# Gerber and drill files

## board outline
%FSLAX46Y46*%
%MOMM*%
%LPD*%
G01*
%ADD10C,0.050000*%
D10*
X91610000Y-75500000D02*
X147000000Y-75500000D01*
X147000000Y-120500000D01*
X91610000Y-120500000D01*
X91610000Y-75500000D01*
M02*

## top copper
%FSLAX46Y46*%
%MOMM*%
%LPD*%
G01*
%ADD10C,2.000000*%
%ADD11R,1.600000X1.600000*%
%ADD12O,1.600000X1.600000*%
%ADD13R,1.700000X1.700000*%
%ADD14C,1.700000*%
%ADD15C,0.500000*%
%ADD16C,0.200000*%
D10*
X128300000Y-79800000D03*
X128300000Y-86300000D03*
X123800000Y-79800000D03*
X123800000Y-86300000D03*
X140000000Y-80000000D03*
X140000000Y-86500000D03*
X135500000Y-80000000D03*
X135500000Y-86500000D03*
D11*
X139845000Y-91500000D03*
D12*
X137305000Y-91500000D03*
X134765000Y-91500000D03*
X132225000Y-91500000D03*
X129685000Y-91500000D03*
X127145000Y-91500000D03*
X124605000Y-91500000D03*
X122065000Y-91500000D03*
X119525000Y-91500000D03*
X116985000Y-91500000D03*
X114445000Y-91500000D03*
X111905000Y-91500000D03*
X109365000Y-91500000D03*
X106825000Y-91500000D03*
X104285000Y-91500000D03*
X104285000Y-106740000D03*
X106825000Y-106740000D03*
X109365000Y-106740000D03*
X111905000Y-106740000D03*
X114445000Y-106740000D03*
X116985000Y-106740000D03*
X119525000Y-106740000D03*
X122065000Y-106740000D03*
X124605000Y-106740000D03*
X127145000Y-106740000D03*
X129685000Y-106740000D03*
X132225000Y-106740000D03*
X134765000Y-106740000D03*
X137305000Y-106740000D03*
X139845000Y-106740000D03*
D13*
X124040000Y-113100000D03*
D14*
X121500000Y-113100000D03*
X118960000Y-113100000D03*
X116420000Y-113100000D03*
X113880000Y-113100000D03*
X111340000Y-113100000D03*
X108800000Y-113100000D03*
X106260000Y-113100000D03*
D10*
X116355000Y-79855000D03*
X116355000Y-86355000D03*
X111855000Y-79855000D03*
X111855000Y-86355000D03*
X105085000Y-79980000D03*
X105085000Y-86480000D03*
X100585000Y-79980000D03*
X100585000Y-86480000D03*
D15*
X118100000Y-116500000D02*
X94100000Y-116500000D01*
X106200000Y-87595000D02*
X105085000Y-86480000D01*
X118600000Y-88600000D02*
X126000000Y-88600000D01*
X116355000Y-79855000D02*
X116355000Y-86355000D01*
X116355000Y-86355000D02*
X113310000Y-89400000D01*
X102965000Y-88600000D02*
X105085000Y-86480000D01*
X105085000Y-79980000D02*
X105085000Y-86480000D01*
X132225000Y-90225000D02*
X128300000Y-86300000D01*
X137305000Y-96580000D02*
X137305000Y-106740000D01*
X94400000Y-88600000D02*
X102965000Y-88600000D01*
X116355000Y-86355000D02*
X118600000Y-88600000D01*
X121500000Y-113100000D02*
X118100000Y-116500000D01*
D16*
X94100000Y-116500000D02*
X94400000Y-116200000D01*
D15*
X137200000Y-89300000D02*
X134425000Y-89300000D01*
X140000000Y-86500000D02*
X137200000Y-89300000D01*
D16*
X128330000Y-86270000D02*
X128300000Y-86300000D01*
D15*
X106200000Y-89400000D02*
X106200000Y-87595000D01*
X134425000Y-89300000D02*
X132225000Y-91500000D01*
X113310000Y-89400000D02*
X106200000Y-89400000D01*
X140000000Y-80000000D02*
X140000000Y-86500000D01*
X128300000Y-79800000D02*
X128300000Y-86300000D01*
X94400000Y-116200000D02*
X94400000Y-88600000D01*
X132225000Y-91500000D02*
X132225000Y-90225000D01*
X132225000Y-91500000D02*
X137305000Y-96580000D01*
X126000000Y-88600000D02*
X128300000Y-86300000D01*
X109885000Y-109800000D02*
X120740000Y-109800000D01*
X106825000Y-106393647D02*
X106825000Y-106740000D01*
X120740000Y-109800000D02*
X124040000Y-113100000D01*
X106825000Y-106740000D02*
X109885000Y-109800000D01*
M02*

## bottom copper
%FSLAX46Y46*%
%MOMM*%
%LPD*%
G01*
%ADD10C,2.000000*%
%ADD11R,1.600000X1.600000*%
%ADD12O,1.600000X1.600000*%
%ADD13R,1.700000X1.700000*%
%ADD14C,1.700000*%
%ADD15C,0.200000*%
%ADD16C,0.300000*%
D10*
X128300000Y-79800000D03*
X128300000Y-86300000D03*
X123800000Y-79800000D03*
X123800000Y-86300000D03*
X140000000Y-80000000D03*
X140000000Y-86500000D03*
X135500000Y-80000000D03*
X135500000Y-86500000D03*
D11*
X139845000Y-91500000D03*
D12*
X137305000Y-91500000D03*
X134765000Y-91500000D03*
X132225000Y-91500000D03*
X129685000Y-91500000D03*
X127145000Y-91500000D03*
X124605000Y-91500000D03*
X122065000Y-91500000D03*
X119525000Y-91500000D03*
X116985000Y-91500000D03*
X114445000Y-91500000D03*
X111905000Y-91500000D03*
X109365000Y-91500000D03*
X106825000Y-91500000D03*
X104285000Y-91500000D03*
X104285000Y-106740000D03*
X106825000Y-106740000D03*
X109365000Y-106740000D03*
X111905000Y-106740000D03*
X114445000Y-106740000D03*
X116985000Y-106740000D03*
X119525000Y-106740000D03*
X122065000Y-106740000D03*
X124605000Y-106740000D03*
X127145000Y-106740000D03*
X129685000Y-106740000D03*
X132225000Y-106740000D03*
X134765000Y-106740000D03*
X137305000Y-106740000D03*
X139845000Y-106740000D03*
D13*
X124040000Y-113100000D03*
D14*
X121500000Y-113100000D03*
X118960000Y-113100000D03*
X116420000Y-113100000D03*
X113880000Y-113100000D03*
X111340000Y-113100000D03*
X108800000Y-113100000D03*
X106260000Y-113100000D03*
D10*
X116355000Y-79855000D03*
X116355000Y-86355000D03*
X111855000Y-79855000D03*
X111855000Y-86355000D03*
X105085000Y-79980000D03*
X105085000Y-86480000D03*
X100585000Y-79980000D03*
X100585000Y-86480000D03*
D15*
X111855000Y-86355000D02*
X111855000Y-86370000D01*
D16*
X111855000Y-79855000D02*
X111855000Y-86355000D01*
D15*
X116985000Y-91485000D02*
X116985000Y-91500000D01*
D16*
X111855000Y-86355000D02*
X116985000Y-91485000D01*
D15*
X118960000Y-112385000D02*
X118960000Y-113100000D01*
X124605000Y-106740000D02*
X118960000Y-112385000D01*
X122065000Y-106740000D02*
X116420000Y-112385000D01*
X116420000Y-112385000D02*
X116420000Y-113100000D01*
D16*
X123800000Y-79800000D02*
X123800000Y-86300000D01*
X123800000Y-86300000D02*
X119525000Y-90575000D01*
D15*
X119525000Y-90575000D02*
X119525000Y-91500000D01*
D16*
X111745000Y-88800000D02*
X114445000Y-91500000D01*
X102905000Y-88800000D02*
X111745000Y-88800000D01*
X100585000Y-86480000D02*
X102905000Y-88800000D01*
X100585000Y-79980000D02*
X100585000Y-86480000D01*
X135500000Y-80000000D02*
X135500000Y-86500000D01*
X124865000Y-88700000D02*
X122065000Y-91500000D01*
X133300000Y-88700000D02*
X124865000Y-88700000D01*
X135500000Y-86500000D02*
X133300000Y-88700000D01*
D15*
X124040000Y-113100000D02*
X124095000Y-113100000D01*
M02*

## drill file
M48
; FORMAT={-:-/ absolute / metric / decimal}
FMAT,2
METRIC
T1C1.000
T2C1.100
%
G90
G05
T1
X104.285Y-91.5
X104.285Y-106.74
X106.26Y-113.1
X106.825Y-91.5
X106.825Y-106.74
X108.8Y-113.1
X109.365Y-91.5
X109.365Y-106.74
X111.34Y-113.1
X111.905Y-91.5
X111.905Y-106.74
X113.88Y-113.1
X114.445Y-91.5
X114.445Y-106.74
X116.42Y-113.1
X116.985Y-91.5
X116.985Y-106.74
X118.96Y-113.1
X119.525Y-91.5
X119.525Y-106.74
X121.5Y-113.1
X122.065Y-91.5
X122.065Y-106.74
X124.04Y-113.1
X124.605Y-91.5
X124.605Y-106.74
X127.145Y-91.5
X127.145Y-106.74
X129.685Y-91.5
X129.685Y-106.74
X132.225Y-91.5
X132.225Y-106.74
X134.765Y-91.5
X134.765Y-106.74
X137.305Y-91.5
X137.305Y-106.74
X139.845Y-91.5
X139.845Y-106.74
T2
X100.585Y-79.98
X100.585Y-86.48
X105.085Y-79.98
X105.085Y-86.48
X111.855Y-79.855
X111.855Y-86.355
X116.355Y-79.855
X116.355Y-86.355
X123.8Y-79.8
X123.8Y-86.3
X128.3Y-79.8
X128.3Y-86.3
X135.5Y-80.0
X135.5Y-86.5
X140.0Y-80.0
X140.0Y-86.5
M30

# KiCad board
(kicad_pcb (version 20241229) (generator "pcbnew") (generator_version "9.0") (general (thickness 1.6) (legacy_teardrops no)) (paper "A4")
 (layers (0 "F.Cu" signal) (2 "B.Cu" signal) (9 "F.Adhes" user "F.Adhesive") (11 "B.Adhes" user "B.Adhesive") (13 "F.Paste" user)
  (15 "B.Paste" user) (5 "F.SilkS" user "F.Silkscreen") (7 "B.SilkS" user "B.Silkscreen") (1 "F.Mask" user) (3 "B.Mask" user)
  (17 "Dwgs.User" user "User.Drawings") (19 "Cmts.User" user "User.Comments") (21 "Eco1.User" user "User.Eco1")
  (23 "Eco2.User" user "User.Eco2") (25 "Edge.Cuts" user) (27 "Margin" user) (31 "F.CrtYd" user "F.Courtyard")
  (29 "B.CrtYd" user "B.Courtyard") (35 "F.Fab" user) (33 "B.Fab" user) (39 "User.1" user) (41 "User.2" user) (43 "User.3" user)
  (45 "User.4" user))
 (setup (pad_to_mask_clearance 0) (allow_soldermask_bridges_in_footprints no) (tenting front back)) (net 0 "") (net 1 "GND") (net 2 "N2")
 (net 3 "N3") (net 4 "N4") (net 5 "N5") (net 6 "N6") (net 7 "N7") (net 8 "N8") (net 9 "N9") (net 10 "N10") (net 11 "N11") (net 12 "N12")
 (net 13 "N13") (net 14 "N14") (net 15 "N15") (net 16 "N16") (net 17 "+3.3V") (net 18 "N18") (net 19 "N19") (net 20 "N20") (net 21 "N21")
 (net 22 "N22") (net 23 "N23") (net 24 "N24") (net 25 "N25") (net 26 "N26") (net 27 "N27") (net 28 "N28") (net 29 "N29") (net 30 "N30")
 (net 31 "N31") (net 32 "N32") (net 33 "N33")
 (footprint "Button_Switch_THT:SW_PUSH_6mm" (layer "F.Cu") (at 128.3 79.8 -90)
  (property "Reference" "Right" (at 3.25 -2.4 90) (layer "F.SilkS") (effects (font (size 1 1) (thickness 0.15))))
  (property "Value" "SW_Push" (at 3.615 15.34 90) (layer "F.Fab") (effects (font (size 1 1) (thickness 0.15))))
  (pad "1" thru_hole circle (at 0 0) (size 2 2) (drill 1.1) (layers "*.Cu" "*.Mask") (remove_unused_layers no) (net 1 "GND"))
  (pad "1" thru_hole circle (at 6.5 0) (size 2 2) (drill 1.1) (layers "*.Cu" "*.Mask") (remove_unused_layers no) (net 1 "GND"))
  (pad "2" thru_hole circle (at 0 4.5) (size 2 2) (drill 1.1) (layers "*.Cu" "*.Mask") (remove_unused_layers no) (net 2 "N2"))
  (pad "2" thru_hole circle (at 6.5 4.5) (size 2 2) (drill 1.1) (layers "*.Cu" "*.Mask") (remove_unused_layers no) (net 2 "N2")))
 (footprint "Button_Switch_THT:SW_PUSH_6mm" (layer "F.Cu") (at 140 80 -90)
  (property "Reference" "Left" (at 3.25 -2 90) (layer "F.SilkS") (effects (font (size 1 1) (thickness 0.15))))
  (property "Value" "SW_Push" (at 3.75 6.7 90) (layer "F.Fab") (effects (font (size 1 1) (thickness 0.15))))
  (pad "1" thru_hole circle (at 0 0) (size 2 2) (drill 1.1) (layers "*.Cu" "*.Mask") (remove_unused_layers no) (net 1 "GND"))
  (pad "1" thru_hole circle (at 6.5 0) (size 2 2) (drill 1.1) (layers "*.Cu" "*.Mask") (remove_unused_layers no) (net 1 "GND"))
  (pad "2" thru_hole circle (at 0 4.5) (size 2 2) (drill 1.1) (layers "*.Cu" "*.Mask") (remove_unused_layers no) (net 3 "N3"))
  (pad "2" thru_hole circle (at 6.5 4.5) (size 2 2) (drill 1.1) (layers "*.Cu" "*.Mask") (remove_unused_layers no) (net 3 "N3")))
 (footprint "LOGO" (layer "F.Cu") (at 135.8138 114.7318)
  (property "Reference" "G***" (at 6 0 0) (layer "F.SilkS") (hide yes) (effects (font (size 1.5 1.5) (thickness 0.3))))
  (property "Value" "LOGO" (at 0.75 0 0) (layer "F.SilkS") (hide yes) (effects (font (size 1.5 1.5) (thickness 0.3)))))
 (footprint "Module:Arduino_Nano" (layer "F.Cu") (at 139.845 91.5 -90)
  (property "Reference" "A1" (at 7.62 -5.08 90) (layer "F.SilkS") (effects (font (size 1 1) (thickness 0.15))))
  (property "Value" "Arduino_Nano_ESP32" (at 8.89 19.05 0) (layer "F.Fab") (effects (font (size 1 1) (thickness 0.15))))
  (pad "1" thru_hole rect (at 0 0 270) (size 1.6 1.6) (drill 1) (layers "*.Cu" "*.Mask") (remove_unused_layers no) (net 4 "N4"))
  (pad "2" thru_hole oval (at 0 2.54 270) (size 1.6 1.6) (drill 1) (layers "*.Cu" "*.Mask") (remove_unused_layers no) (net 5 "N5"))
  (pad "3" thru_hole oval (at 0 5.08 270) (size 1.6 1.6) (drill 1) (layers "*.Cu" "*.Mask") (remove_unused_layers no) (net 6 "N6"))
  (pad "4" thru_hole oval (at 0 7.62 270) (size 1.6 1.6) (drill 1) (layers "*.Cu" "*.Mask") (remove_unused_layers no) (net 1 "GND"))
  (pad "5" thru_hole oval (at 0 10.16 270) (size 1.6 1.6) (drill 1) (layers "*.Cu" "*.Mask") (remove_unused_layers no) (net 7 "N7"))
  (pad "6" thru_hole oval (at 0 12.7 270) (size 1.6 1.6) (drill 1) (layers "*.Cu" "*.Mask") (remove_unused_layers no) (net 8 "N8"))
  (pad "7" thru_hole oval (at 0 15.24 270) (size 1.6 1.6) (drill 1) (layers "*.Cu" "*.Mask") (remove_unused_layers no) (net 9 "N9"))
  (pad "8" thru_hole oval (at 0 17.78 270) (size 1.6 1.6) (drill 1) (layers "*.Cu" "*.Mask") (remove_unused_layers no) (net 3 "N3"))
  (pad "9" thru_hole oval (at 0 20.32 270) (size 1.6 1.6) (drill 1) (layers "*.Cu" "*.Mask") (remove_unused_layers no) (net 2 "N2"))
  (pad "10" thru_hole oval (at 0 22.86 270) (size 1.6 1.6) (drill 1) (layers "*.Cu" "*.Mask") (remove_unused_layers no) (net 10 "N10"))
  (pad "11" thru_hole oval (at 0 25.4 270) (size 1.6 1.6) (drill 1) (layers "*.Cu" "*.Mask") (remove_unused_layers no) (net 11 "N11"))
  (pad "12" thru_hole oval (at 0 27.94 270) (size 1.6 1.6) (drill 1) (layers "*.Cu" "*.Mask") (remove_unused_layers no) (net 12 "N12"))
  (pad "13" thru_hole oval (at 0 30.48 270) (size 1.6 1.6) (drill 1) (layers "*.Cu" "*.Mask") (remove_unused_layers no) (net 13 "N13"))
  (pad "14" thru_hole oval (at 0 33.02 270) (size 1.6 1.6) (drill 1) (layers "*.Cu" "*.Mask") (remove_unused_layers no) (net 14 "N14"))
  (pad "15" thru_hole oval (at 0 35.56 270) (size 1.6 1.6) (drill 1) (layers "*.Cu" "*.Mask") (remove_unused_layers no) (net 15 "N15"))
  (pad "16" thru_hole oval (at 15.24 35.56 270) (size 1.6 1.6) (drill 1) (layers "*.Cu" "*.Mask") (remove_unused_layers no) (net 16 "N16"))
  (pad "17" thru_hole oval (at 15.24 33.02 270) (size 1.6 1.6) (drill 1) (layers "*.Cu" "*.Mask") (remove_unused_layers no) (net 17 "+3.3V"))
  (pad "18" thru_hole oval (at 15.24 30.48 270) (size 1.6 1.6) (drill 1) (layers "*.Cu" "*.Mask") (remove_unused_layers no) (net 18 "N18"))
  (pad "19" thru_hole oval (at 15.24 27.94 270) (size 1.6 1.6) (drill 1) (layers "*.Cu" "*.Mask") (remove_unused_layers no) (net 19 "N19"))
  (pad "20" thru_hole oval (at 15.24 25.4 270) (size 1.6 1.6) (drill 1) (layers "*.Cu" "*.Mask") (remove_unused_layers no) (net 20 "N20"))
  (pad "21" thru_hole oval (at 15.24 22.86 270) (size 1.6 1.6) (drill 1) (layers "*.Cu" "*.Mask") (remove_unused_layers no) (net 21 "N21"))
  (pad "22" thru_hole oval (at 15.24 20.32 270) (size 1.6 1.6) (drill 1) (layers "*.Cu" "*.Mask") (remove_unused_layers no) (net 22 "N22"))
  (pad "23" thru_hole oval (at 15.24 17.78 270) (size 1.6 1.6) (drill 1) (layers "*.Cu" "*.Mask") (remove_unused_layers no) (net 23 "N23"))
  (pad "24" thru_hole oval (at 15.24 15.24 270) (size 1.6 1.6) (drill 1) (layers "*.Cu" "*.Mask") (remove_unused_layers no) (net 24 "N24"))
  (pad "25" thru_hole oval (at 15.24 12.7 270) (size 1.6 1.6) (drill 1) (layers "*.Cu" "*.Mask") (remove_unused_layers no) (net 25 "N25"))
  (pad "26" thru_hole oval (at 15.24 10.16 270) (size 1.6 1.6) (drill 1) (layers "*.Cu" "*.Mask") (remove_unused_layers no) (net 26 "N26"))
  (pad "27" thru_hole oval (at 15.24 7.62 270) (size 1.6 1.6) (drill 1) (layers "*.Cu" "*.Mask") (remove_unused_layers no) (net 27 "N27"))
  (pad "28" thru_hole oval (at 15.24 5.08 270) (size 1.6 1.6) (drill 1) (layers "*.Cu" "*.Mask") (remove_unused_layers no) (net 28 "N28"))
  (pad "29" thru_hole oval (at 15.24 2.54 270) (size 1.6 1.6) (drill 1) (layers "*.Cu" "*.Mask") (remove_unused_layers no) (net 1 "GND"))
  (pad "30" thru_hole oval (at 15.24 0 270) (size 1.6 1.6) (drill 1) (layers "*.Cu" "*.Mask") (remove_unused_layers no) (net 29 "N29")))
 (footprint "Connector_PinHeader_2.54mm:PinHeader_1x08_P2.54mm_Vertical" (layer "F.Cu") (at 124.04 113.1 -90)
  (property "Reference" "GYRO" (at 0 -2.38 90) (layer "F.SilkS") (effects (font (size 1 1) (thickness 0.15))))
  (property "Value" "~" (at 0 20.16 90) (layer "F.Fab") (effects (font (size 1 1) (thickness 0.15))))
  (pad "1" thru_hole rect (at 0 0 270) (size 1.7 1.7) (drill 1) (layers "*.Cu" "*.Mask") (remove_unused_layers no) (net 17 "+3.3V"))
  (pad "2" thru_hole circle (at 0 2.54 270) (size 1.7 1.7) (drill 1) (layers "*.Cu" "*.Mask") (remove_unused_layers no) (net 1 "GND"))
  (pad "3" thru_hole circle (at 0 5.08 270) (size 1.7 1.7) (drill 1) (layers "*.Cu" "*.Mask") (remove_unused_layers no) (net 24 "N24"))
  (pad "4" thru_hole circle (at 0 7.62 270) (size 1.7 1.7) (drill 1) (layers "*.Cu" "*.Mask") (remove_unused_layers no) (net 23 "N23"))
  (pad "5" thru_hole circle (at 0 10.16 270) (size 1.7 1.7) (drill 1) (layers "*.Cu" "*.Mask") (remove_unused_layers no) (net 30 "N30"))
  (pad "6" thru_hole circle (at 0 12.7 270) (size 1.7 1.7) (drill 1) (layers "*.Cu" "*.Mask") (remove_unused_layers no) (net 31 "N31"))
  (pad "7" thru_hole circle (at 0 15.24 270) (size 1.7 1.7) (drill 1) (layers "*.Cu" "*.Mask") (remove_unused_layers no) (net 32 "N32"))
  (pad "8" thru_hole circle (at 0 17.78 270) (size 1.7 1.7) (drill 1) (layers "*.Cu" "*.Mask") (remove_unused_layers no) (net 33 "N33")))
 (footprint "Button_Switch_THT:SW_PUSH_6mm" (layer "F.Cu") (at 116.355 79.855 -90)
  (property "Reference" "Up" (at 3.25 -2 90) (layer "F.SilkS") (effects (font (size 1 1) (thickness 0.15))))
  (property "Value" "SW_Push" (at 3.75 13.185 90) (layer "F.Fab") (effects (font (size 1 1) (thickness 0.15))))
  (pad "1" thru_hole circle (at 0 0) (size 2 2) (drill 1.1) (layers "*.Cu" "*.Mask") (remove_unused_layers no) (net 1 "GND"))
  (pad "1" thru_hole circle (at 6.5 0) (size 2 2) (drill 1.1) (layers "*.Cu" "*.Mask") (remove_unused_layers no) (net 1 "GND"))
  (pad "2" thru_hole circle (at 0 4.5) (size 2 2) (drill 1.1) (layers "*.Cu" "*.Mask") (remove_unused_layers no) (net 10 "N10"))
  (pad "2" thru_hole circle (at 6.5 4.5) (size 2 2) (drill 1.1) (layers "*.Cu" "*.Mask") (remove_unused_layers no) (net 10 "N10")))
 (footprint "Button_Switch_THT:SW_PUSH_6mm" (layer "F.Cu") (at 105.085 79.98 -90)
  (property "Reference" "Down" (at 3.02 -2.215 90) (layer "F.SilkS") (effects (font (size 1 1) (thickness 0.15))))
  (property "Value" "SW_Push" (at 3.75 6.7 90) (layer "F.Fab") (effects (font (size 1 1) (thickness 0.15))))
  (pad "1" thru_hole circle (at 0 0) (size 2 2) (drill 1.1) (layers "*.Cu" "*.Mask") (remove_unused_layers no) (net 1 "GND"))
  (pad "1" thru_hole circle (at 6.5 0) (size 2 2) (drill 1.1) (layers "*.Cu" "*.Mask") (remove_unused_layers no) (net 1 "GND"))
  (pad "2" thru_hole circle (at 0 4.5) (size 2 2) (drill 1.1) (layers "*.Cu" "*.Mask") (remove_unused_layers no) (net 11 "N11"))
  (pad "2" thru_hole circle (at 6.5 4.5) (size 2 2) (drill 1.1) (layers "*.Cu" "*.Mask") (remove_unused_layers no) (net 11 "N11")))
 (gr_rect (start 91.61 75.5) (end 147 120.5) (stroke (width 0.05) (type solid)) (fill no) (layer "Edge.Cuts"))
 (segment (start 111.855 86.355) (end 111.855 86.37) (width 0.2) (layer "B.Cu") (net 10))
 (segment (start 111.855 79.855) (end 111.855 86.355) (width 0.3) (layer "B.Cu") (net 10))
 (segment (start 116.985 91.485) (end 116.985 91.5) (width 0.2) (layer "B.Cu") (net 10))
 (segment (start 111.855 86.355) (end 116.985 91.485) (width 0.3) (layer "B.Cu") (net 10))
 (segment (start 118.96 112.385) (end 118.96 113.1) (width 0.2) (layer "B.Cu") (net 24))
 (segment (start 124.605 106.74) (end 118.96 112.385) (width 0.2) (layer "B.Cu") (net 24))
 (segment (start 122.065 106.74) (end 116.42 112.385) (width 0.2) (layer "B.Cu") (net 23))
 (segment (start 116.42 112.385) (end 116.42 113.1) (width 0.2) (layer "B.Cu") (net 23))
 (segment (start 123.8 79.8) (end 123.8 86.3) (width 0.3) (layer "B.Cu") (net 2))
 (segment (start 123.8 86.3) (end 119.525 90.575) (width 0.3) (layer "B.Cu") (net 2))
 (segment (start 119.525 90.575) (end 119.525 91.5) (width 0.2) (layer "B.Cu") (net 2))
 (segment (start 118.1 116.5) (end 94.1 116.5) (width 0.5) (layer "F.Cu") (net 1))
 (segment (start 106.2 87.595) (end 105.085 86.48) (width 0.5) (layer "F.Cu") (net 1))
 (segment (start 118.6 88.6) (end 126 88.6) (width 0.5) (layer "F.Cu") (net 1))
 (segment (start 116.355 79.855) (end 116.355 86.355) (width 0.5) (layer "F.Cu") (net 1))
 (segment (start 116.355 86.355) (end 113.31 89.4) (width 0.5) (layer "F.Cu") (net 1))
 (segment (start 102.965 88.6) (end 105.085 86.48) (width 0.5) (layer "F.Cu") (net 1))
 (segment (start 105.085 79.98) (end 105.085 86.48) (width 0.5) (layer "F.Cu") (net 1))
 (segment (start 132.225 90.225) (end 128.3 86.3) (width 0.5) (layer "F.Cu") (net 1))
 (segment (start 137.305 96.58) (end 137.305 106.74) (width 0.5) (layer "F.Cu") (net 1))
 (segment (start 94.4 88.6) (end 102.965 88.6) (width 0.5) (layer "F.Cu") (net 1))
 (segment (start 116.355 86.355) (end 118.6 88.6) (width 0.5) (layer "F.Cu") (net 1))
 (segment (start 121.5 113.1) (end 118.1 116.5) (width 0.5) (layer "F.Cu") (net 1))
 (segment (start 94.1 116.5) (end 94.4 116.2) (width 0.2) (layer "F.Cu") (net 1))
 (segment (start 137.2 89.3) (end 134.425 89.3) (width 0.5) (layer "F.Cu") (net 1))
 (segment (start 140 86.5) (end 137.2 89.3) (width 0.5) (layer "F.Cu") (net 1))
 (segment (start 128.33 86.27) (end 128.3 86.3) (width 0.2) (layer "F.Cu") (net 1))
 (segment (start 106.2 89.4) (end 106.2 87.595) (width 0.5) (layer "F.Cu") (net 1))
 (segment (start 134.425 89.3) (end 132.225 91.5) (width 0.5) (layer "F.Cu") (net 1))
 (segment (start 113.31 89.4) (end 106.2 89.4) (width 0.5) (layer "F.Cu") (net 1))
 (segment (start 140 80) (end 140 86.5) (width 0.5) (layer "F.Cu") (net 1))
 (segment (start 128.3 79.8) (end 128.3 86.3) (width 0.5) (layer "F.Cu") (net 1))
 (segment (start 94.4 116.2) (end 94.4 88.6) (width 0.5) (layer "F.Cu") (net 1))
 (segment (start 132.225 91.5) (end 132.225 90.225) (width 0.5) (layer "F.Cu") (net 1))
 (segment (start 132.225 91.5) (end 137.305 96.58) (width 0.5) (layer "F.Cu") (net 1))
 (segment (start 126 88.6) (end 128.3 86.3) (width 0.5) (layer "F.Cu") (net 1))
 (segment (start 111.745 88.8) (end 114.445 91.5) (width 0.3) (layer "B.Cu") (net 11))
 (segment (start 102.905 88.8) (end 111.745 88.8) (width 0.3) (layer "B.Cu") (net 11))
 (segment (start 100.585 86.48) (end 102.905 88.8) (width 0.3) (layer "B.Cu") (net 11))
 (segment (start 100.585 79.98) (end 100.585 86.48) (width 0.3) (layer "B.Cu") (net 11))
 (segment (start 135.5 80) (end 135.5 86.5) (width 0.3) (layer "B.Cu") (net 3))
 (segment (start 124.865 88.7) (end 122.065 91.5) (width 0.3) (layer "B.Cu") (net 3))
 (segment (start 133.3 88.7) (end 124.865 88.7) (width 0.3) (layer "B.Cu") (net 3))
 (segment (start 135.5 86.5) (end 133.3 88.7) (width 0.3) (layer "B.Cu") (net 3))
 (segment (start 109.885 109.8) (end 120.74 109.8) (width 0.5) (layer "F.Cu") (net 17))
 (segment (start 106.825 106.393647) (end 106.825 106.74) (width 0.5) (layer "F.Cu") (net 17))
 (segment (start 120.74 109.8) (end 124.04 113.1) (width 0.5) (layer "F.Cu") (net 17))
 (segment (start 106.825 106.74) (end 109.885 109.8) (width 0.5) (layer "F.Cu") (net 17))
 (segment (start 124.04 113.1) (end 124.095 113.1) (width 0.2) (layer "B.Cu") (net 17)))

